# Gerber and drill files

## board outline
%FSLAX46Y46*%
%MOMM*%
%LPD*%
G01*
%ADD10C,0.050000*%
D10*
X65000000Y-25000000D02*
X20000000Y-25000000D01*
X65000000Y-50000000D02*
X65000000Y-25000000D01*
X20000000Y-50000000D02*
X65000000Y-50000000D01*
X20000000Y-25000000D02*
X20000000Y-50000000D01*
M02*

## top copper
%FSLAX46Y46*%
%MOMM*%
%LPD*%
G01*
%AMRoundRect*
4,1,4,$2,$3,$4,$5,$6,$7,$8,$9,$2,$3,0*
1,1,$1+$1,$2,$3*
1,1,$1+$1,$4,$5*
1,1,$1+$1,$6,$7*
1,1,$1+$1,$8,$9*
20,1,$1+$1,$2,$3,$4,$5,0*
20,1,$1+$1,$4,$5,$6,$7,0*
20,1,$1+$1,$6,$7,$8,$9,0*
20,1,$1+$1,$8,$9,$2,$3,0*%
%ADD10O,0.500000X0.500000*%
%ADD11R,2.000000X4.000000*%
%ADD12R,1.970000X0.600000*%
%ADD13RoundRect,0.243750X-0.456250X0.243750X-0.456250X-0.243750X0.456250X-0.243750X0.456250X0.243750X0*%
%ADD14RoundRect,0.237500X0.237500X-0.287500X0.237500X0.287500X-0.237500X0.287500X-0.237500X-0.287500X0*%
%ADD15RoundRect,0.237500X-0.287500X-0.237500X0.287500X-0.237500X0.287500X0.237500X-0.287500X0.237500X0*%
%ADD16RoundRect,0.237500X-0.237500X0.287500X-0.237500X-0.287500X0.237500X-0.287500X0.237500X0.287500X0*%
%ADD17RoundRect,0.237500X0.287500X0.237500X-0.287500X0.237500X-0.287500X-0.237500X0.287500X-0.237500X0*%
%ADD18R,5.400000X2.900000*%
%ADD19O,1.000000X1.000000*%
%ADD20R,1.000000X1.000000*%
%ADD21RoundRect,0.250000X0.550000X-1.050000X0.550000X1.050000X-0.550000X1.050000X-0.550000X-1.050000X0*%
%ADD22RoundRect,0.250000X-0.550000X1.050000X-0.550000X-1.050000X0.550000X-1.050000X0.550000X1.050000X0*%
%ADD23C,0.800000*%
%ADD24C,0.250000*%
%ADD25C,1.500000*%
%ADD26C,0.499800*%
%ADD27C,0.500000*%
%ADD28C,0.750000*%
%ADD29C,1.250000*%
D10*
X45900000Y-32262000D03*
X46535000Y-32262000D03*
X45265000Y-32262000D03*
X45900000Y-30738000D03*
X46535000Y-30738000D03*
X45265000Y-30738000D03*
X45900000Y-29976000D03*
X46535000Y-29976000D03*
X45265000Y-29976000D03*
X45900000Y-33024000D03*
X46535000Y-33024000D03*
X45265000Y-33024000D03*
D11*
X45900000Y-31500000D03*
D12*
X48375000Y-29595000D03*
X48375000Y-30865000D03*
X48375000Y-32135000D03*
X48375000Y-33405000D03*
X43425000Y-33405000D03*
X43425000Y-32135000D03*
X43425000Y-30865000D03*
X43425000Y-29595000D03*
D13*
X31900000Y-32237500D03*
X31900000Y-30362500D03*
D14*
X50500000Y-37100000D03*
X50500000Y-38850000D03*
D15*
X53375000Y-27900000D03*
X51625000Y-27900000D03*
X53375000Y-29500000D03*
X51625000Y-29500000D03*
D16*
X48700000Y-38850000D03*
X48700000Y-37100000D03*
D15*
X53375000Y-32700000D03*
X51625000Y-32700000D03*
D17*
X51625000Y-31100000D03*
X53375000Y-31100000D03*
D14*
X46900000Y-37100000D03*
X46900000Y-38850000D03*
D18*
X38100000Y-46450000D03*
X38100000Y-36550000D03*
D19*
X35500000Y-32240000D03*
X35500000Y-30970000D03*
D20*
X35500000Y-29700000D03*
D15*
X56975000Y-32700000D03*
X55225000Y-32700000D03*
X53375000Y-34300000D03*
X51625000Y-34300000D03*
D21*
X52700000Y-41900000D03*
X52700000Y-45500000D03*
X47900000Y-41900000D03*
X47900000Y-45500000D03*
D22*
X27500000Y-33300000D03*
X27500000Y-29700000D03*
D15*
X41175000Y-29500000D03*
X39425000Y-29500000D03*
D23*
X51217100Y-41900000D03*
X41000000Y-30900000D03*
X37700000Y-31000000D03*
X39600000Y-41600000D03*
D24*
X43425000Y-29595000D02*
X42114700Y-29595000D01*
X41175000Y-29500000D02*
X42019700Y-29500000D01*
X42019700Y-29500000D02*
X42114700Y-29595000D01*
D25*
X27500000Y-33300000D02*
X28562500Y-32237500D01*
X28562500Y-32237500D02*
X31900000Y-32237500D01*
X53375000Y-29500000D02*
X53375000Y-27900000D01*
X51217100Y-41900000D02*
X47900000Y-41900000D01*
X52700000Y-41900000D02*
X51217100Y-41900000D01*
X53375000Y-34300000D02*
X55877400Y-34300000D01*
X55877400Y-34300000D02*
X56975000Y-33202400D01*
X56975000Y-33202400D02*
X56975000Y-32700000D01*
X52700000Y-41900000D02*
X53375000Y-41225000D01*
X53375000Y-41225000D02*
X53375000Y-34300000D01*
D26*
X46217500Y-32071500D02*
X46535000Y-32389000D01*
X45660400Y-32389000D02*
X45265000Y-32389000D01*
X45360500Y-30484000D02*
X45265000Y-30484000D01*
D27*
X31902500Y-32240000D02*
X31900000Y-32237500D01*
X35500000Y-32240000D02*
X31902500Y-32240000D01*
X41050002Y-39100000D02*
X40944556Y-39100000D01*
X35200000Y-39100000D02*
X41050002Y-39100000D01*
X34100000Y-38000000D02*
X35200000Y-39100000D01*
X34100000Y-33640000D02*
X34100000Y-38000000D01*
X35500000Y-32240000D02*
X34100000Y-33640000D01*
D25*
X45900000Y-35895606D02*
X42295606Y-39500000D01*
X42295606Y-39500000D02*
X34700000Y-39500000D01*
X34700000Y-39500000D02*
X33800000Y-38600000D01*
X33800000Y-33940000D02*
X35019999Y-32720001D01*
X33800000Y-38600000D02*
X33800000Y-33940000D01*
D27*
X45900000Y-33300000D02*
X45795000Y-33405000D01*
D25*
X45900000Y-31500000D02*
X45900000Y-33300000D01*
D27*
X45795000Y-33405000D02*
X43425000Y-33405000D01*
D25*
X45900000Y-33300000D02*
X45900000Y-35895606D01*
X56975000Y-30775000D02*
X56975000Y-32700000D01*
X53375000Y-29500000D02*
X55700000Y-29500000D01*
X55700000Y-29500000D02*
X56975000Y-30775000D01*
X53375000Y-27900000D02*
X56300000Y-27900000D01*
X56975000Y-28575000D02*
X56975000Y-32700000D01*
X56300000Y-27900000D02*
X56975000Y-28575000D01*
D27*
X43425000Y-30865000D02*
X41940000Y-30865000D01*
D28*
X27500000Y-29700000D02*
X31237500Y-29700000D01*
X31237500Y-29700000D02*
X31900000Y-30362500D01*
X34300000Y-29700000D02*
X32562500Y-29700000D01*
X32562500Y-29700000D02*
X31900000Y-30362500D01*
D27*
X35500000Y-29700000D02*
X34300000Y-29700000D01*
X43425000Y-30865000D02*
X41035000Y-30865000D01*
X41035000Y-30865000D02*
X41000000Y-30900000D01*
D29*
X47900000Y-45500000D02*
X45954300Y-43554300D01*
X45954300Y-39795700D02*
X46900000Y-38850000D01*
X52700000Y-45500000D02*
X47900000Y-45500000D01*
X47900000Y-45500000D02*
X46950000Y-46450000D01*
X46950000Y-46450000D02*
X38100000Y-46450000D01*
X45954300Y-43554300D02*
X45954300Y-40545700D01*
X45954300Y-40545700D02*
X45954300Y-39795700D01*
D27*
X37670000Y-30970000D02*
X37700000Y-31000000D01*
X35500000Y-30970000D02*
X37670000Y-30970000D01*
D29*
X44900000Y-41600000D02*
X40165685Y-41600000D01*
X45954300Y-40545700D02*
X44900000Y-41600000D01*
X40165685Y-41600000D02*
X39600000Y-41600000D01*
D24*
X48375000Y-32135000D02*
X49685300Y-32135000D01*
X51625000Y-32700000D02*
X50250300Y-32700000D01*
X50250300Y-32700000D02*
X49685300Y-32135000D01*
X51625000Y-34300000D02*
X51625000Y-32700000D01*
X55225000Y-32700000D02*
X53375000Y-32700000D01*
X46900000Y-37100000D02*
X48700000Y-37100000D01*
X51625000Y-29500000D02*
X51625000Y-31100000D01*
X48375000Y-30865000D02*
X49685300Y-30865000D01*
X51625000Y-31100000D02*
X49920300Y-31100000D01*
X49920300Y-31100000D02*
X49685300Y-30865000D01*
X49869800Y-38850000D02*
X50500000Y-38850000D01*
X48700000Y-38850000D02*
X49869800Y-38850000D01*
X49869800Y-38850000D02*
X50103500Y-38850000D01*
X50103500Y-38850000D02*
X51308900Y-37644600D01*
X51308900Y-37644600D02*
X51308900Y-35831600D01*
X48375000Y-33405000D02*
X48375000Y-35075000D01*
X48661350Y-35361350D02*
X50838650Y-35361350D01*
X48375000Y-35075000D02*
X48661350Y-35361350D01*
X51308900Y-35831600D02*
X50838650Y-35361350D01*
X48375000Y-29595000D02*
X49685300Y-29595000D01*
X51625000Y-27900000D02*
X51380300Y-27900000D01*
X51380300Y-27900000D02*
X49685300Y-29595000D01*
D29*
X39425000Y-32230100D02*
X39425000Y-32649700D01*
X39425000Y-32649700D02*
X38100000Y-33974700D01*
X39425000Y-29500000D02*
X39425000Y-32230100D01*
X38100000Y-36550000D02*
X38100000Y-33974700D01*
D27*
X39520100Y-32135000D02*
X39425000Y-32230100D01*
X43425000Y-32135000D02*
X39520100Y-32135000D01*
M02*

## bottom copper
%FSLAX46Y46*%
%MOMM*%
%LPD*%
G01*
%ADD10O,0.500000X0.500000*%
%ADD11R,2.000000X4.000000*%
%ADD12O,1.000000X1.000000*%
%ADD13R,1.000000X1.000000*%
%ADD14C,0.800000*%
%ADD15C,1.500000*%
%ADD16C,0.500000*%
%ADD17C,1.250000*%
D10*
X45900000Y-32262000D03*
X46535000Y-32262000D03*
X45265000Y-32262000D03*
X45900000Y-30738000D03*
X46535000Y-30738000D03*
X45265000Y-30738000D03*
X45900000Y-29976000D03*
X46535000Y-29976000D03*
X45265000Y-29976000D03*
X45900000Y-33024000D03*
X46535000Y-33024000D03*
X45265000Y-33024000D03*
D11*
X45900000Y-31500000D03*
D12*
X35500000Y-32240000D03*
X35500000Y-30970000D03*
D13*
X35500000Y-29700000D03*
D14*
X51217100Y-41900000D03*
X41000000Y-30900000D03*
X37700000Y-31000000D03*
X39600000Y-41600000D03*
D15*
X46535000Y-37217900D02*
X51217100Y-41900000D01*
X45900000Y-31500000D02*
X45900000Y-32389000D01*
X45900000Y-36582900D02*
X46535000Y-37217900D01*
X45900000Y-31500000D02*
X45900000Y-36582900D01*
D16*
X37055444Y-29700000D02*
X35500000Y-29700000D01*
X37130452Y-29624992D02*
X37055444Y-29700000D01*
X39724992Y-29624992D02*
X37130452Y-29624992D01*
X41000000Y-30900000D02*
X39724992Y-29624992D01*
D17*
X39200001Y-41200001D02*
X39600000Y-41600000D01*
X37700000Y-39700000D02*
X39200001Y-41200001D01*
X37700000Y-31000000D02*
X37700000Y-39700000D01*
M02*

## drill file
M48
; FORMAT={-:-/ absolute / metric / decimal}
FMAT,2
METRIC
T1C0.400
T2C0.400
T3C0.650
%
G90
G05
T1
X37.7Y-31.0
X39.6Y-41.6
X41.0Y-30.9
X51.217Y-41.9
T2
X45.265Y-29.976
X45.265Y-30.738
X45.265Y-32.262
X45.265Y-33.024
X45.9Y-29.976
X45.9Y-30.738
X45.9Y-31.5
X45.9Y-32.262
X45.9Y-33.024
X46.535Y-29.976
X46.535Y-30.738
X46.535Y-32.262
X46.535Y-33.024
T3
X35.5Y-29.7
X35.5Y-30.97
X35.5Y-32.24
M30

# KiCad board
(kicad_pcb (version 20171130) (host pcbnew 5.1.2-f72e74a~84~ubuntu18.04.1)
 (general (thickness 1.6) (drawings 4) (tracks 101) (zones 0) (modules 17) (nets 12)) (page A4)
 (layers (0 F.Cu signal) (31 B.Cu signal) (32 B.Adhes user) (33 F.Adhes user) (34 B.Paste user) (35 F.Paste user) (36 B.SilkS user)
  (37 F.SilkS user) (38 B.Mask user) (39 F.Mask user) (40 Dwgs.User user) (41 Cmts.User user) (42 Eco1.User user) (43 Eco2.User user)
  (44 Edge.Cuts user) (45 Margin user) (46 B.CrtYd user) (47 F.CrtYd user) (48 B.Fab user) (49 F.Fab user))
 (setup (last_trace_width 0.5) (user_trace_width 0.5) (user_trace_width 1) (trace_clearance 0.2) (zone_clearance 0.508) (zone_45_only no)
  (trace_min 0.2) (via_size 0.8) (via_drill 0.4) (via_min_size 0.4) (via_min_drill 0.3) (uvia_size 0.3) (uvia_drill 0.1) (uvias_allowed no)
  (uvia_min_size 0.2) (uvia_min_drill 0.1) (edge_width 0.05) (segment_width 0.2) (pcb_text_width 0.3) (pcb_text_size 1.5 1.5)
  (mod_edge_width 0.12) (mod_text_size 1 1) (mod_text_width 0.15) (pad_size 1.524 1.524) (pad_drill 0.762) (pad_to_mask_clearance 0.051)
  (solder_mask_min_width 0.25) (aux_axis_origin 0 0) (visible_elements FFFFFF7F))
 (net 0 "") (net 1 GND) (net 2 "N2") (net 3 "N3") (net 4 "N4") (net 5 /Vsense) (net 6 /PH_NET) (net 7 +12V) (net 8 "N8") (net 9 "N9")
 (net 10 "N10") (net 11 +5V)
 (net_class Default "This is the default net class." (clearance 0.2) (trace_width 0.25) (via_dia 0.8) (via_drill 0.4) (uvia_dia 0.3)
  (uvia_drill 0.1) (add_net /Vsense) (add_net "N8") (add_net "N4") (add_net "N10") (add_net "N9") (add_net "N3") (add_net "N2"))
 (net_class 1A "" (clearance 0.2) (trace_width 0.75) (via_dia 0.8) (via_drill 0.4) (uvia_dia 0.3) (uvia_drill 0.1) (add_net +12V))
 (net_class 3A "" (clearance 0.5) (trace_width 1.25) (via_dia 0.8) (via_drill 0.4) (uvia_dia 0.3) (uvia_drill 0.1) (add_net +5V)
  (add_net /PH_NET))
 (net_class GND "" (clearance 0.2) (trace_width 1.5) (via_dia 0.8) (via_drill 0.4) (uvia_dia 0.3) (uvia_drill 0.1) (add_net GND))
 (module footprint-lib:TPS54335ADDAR (layer F.Cu) (at 45.9 31.5)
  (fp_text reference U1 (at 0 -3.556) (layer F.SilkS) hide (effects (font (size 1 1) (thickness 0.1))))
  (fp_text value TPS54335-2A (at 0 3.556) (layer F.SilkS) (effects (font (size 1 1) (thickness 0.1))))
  (pad PAD thru_hole oval (at 0 0.762) (size 0.5 0.5) (drill 0.4) (layers *.Cu F.Mask) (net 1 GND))
  (pad PAD thru_hole oval (at 0.635 0.762) (size 0.5 0.5) (drill 0.4) (layers *.Cu F.Mask) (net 1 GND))
  (pad PAD thru_hole oval (at -0.635 0.762) (size 0.5 0.5) (drill 0.4) (layers *.Cu F.Mask) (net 1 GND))
  (pad PAD thru_hole oval (at 0 -0.762) (size 0.5 0.5) (drill 0.4) (layers *.Cu F.Mask) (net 1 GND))
  (pad PAD thru_hole oval (at 0.635 -0.762) (size 0.5 0.5) (drill 0.4) (layers *.Cu F.Mask) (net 1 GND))
  (pad PAD thru_hole oval (at -0.635 -0.762) (size 0.5 0.5) (drill 0.4) (layers *.Cu F.Mask) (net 1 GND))
  (pad PAD thru_hole oval (at 0 -1.524) (size 0.5 0.5) (drill 0.4) (layers *.Cu F.Mask) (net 1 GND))
  (pad PAD thru_hole oval (at 0.635 -1.524) (size 0.5 0.5) (drill 0.4) (layers *.Cu F.Mask) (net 1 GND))
  (pad PAD thru_hole oval (at -0.635 -1.524) (size 0.5 0.5) (drill 0.4) (layers *.Cu F.Mask) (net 1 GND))
  (pad PAD thru_hole oval (at 0 1.524) (size 0.5 0.5) (drill 0.4) (layers *.Cu F.Mask) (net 1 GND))
  (pad PAD thru_hole oval (at 0.635 1.524) (size 0.5 0.5) (drill 0.4) (layers *.Cu F.Mask) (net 1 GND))
  (pad PAD thru_hole oval (at -0.635 1.524) (size 0.5 0.5) (drill 0.4) (layers *.Cu F.Mask) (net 1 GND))
  (pad PAD thru_hole rect (at 0 0) (size 2 4) (drill 0.4) (layers *.Cu F.Paste F.Mask) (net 1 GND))
  (pad 8 smd rect (at 2.475 -1.905) (size 1.97 0.6) (layers F.Cu F.Paste F.Mask) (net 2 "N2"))
  (pad 7 smd rect (at 2.475 -0.635) (size 1.97 0.6) (layers F.Cu F.Paste F.Mask) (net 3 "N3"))
  (pad 6 smd rect (at 2.475 0.635) (size 1.97 0.6) (layers F.Cu F.Paste F.Mask) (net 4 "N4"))
  (pad 5 smd rect (at 2.475 1.905) (size 1.97 0.6) (layers F.Cu F.Paste F.Mask) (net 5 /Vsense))
  (pad 4 smd rect (at -2.475 1.905) (size 1.97 0.6) (layers F.Cu F.Paste F.Mask) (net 1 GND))
  (pad 3 smd rect (at -2.475 0.635) (size 1.97 0.6) (layers F.Cu F.Paste F.Mask) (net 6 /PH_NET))
  (pad 2 smd rect (at -2.475 -0.635) (size 1.97 0.6) (layers F.Cu F.Paste F.Mask) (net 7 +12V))
  (pad 1 smd rect (at -2.475 -1.905) (size 1.97 0.6) (layers F.Cu F.Paste F.Mask) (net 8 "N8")))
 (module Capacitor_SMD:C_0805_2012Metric (layer F.Cu) (at 31.9 31.3 270)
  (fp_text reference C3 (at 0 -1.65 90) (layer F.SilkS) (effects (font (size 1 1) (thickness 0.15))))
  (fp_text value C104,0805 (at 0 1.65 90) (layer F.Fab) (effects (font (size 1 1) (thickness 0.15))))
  (pad 2 smd roundrect (at 0.9375 0 270) (size 0.975 1.4) (layers F.Cu F.Paste F.Mask) (roundrect_rratio 0.25) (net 1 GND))
  (pad 1 smd roundrect (at -0.9375 0 270) (size 0.975 1.4) (layers F.Cu F.Paste F.Mask) (roundrect_rratio 0.25) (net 7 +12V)))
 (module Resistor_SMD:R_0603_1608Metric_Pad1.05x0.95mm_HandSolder (layer F.Cu) (at 50.5 37.975 90)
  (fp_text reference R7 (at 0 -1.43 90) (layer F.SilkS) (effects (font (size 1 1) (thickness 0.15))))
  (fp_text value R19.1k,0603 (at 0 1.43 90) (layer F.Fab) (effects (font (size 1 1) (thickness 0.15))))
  (pad 2 smd roundrect (at 0.875 0 90) (size 1.05 0.95) (layers F.Cu F.Paste F.Mask) (roundrect_rratio 0.25) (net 1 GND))
  (pad 1 smd roundrect (at -0.875 0 90) (size 1.05 0.95) (layers F.Cu F.Paste F.Mask) (roundrect_rratio 0.25) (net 5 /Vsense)))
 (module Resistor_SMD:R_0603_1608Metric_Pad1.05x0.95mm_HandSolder (layer F.Cu) (at 52.5 27.9)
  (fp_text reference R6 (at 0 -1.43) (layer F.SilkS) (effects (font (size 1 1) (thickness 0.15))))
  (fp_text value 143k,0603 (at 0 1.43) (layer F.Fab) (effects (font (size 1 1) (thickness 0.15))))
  (pad 2 smd roundrect (at 0.875 0) (size 1.05 0.95) (layers F.Cu F.Paste F.Mask) (roundrect_rratio 0.25) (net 1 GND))
  (pad 1 smd roundrect (at -0.875 0) (size 1.05 0.95) (layers F.Cu F.Paste F.Mask) (roundrect_rratio 0.25) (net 2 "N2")))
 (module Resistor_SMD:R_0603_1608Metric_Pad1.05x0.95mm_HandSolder (layer F.Cu) (at 52.5 29.5)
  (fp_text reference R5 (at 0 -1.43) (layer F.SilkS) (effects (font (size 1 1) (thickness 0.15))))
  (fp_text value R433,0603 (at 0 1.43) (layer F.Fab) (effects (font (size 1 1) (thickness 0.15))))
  (pad 2 smd roundrect (at 0.875 0) (size 1.05 0.95) (layers F.Cu F.Paste F.Mask) (roundrect_rratio 0.25) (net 1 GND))
  (pad 1 smd roundrect (at -0.875 0) (size 1.05 0.95) (layers F.Cu F.Paste F.Mask) (roundrect_rratio 0.25) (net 3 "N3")))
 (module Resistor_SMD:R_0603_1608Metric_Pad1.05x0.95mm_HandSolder (layer F.Cu) (at 48.7 37.975 270)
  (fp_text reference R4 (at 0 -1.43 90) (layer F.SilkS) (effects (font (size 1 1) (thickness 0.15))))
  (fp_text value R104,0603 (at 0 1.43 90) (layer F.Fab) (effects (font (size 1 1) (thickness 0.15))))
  (pad 2 smd roundrect (at 0.875 0 270) (size 1.05 0.95) (layers F.Cu F.Paste F.Mask) (roundrect_rratio 0.25) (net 5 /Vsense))
  (pad 1 smd roundrect (at -0.875 0 270) (size 1.05 0.95) (layers F.Cu F.Paste F.Mask) (roundrect_rratio 0.25) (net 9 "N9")))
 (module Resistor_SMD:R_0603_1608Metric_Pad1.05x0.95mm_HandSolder (layer F.Cu) (at 52.5 32.7)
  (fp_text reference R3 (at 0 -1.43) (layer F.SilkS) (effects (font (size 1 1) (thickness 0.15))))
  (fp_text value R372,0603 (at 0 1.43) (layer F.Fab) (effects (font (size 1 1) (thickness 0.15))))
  (pad 2 smd roundrect (at 0.875 0) (size 1.05 0.95) (layers F.Cu F.Paste F.Mask) (roundrect_rratio 0.25) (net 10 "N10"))
  (pad 1 smd roundrect (at -0.875 0) (size 1.05 0.95) (layers F.Cu F.Paste F.Mask) (roundrect_rratio 0.25) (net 4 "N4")))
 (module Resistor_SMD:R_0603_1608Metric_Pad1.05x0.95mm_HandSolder (layer F.Cu) (at 52.5 31.1 180)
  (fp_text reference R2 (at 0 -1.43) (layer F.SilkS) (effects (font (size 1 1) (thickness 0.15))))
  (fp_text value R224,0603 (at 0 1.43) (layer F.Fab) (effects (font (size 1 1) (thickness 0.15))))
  (pad 2 smd roundrect (at 0.875 0 180) (size 1.05 0.95) (layers F.Cu F.Paste F.Mask) (roundrect_rratio 0.25) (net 3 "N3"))
  (pad 1 smd roundrect (at -0.875 0 180) (size 1.05 0.95) (layers F.Cu F.Paste F.Mask) (roundrect_rratio 0.25) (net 7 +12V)))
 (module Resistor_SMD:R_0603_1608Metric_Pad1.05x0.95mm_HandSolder (layer F.Cu) (at 46.9 37.975 90)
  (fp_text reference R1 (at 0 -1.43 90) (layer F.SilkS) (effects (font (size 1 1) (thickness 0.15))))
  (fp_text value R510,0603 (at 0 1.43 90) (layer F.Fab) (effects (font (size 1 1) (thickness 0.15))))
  (pad 2 smd roundrect (at 0.875 0 90) (size 1.05 0.95) (layers F.Cu F.Paste F.Mask) (roundrect_rratio 0.25) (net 9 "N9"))
  (pad 1 smd roundrect (at -0.875 0 90) (size 1.05 0.95) (layers F.Cu F.Paste F.Mask) (roundrect_rratio 0.25) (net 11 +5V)))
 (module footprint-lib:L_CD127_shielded (layer F.Cu) (at 38.1 41.5 270)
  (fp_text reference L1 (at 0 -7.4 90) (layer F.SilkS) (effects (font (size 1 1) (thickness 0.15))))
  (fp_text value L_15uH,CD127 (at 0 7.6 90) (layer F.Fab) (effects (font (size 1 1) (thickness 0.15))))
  (pad 2 smd rect (at 4.95 0 270) (size 2.9 5.4) (layers F.Cu F.Paste F.Mask) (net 11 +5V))
  (pad 1 smd rect (at -4.95 0 270) (size 2.9 5.4) (layers F.Cu F.Paste F.Mask) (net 6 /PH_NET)))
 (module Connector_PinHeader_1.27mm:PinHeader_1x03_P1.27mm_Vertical (layer F.Cu) (at 35.5 29.7)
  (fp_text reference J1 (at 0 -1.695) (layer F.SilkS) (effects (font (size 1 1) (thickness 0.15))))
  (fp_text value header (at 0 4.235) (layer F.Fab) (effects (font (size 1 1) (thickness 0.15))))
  (pad 3 thru_hole oval (at 0 2.54) (size 1 1) (drill 0.65) (layers *.Cu *.Mask) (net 1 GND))
  (pad 2 thru_hole oval (at 0 1.27) (size 1 1) (drill 0.65) (layers *.Cu *.Mask) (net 11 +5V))
  (pad 1 thru_hole rect (at 0 0) (size 1 1) (drill 0.65) (layers *.Cu *.Mask) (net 7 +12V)))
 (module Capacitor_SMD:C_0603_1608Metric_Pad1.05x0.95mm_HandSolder (layer F.Cu) (at 56.1 32.7)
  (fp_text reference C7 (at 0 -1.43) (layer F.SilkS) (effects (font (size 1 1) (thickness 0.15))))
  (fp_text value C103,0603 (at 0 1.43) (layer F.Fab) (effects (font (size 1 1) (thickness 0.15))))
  (pad 2 smd roundrect (at 0.875 0) (size 1.05 0.95) (layers F.Cu F.Paste F.Mask) (roundrect_rratio 0.25) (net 1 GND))
  (pad 1 smd roundrect (at -0.875 0) (size 1.05 0.95) (layers F.Cu F.Paste F.Mask) (roundrect_rratio 0.25) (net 10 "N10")))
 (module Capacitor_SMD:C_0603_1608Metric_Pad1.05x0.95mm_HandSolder (layer F.Cu) (at 52.5 34.3)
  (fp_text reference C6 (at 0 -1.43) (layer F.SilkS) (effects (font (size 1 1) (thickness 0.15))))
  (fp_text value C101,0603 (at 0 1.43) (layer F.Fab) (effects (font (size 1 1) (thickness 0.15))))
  (pad 2 smd roundrect (at 0.875 0) (size 1.05 0.95) (layers F.Cu F.Paste F.Mask) (roundrect_rratio 0.25) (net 1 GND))
  (pad 1 smd roundrect (at -0.875 0) (size 1.05 0.95) (layers F.Cu F.Paste F.Mask) (roundrect_rratio 0.25) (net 4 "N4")))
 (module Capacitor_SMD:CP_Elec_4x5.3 (layer F.Cu) (at 52.7 43.7 90)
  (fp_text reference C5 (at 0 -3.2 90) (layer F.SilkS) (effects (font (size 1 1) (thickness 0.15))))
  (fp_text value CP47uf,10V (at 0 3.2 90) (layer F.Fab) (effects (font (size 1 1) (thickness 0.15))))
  (pad 2 smd roundrect (at 1.8 0 90) (size 2.6 1.6) (layers F.Cu F.Paste F.Mask) (roundrect_rratio 0.15625) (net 1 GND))
  (pad 1 smd roundrect (at -1.8 0 90) (size 2.6 1.6) (layers F.Cu F.Paste F.Mask) (roundrect_rratio 0.15625) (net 11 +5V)))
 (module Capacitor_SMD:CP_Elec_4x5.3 (layer F.Cu) (at 47.9 43.7 90)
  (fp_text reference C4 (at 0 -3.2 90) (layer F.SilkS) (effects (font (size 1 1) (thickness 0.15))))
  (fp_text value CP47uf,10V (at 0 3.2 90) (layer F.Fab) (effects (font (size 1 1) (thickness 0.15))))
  (pad 2 smd roundrect (at 1.8 0 90) (size 2.6 1.6) (layers F.Cu F.Paste F.Mask) (roundrect_rratio 0.15625) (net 1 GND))
  (pad 1 smd roundrect (at -1.8 0 90) (size 2.6 1.6) (layers F.Cu F.Paste F.Mask) (roundrect_rratio 0.15625) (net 11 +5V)))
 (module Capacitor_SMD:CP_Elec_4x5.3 (layer F.Cu) (at 27.5 31.5 270)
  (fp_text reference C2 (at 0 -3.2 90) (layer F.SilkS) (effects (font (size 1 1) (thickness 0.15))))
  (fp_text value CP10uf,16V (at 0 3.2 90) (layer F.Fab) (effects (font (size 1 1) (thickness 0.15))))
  (pad 2 smd roundrect (at 1.8 0 270) (size 2.6 1.6) (layers F.Cu F.Paste F.Mask) (roundrect_rratio 0.15625) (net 1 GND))
  (pad 1 smd roundrect (at -1.8 0 270) (size 2.6 1.6) (layers F.Cu F.Paste F.Mask) (roundrect_rratio 0.15625) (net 7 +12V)))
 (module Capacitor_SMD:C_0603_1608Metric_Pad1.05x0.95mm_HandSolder (layer F.Cu) (at 40.3 29.5)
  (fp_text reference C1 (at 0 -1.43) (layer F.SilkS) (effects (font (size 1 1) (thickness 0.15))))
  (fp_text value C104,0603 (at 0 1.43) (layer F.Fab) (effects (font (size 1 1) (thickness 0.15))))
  (pad 2 smd roundrect (at 0.875 0) (size 1.05 0.95) (layers F.Cu F.Paste F.Mask) (roundrect_rratio 0.25) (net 8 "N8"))
  (pad 1 smd roundrect (at -0.875 0) (size 1.05 0.95) (layers F.Cu F.Paste F.Mask) (roundrect_rratio 0.25) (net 6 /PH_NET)))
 (gr_line (start 65 25) (end 20 25) (layer Edge.Cuts) (width 0.05))
 (gr_line (start 65 50) (end 65 25) (layer Edge.Cuts) (width 0.05))
 (gr_line (start 20 50) (end 65 50) (layer Edge.Cuts) (width 0.05))
 (gr_line (start 20 25) (end 20 50) (layer Edge.Cuts) (width 0.05))
 (segment (start 43.425 29.595) (end 42.1147 29.595) (width 0.25) (layer F.Cu) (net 8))
 (segment (start 41.175 29.5) (end 42.0197 29.5) (width 0.25) (layer F.Cu) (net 8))
 (segment (start 42.0197 29.5) (end 42.1147 29.595) (width 0.25) (layer F.Cu) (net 8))
 (segment (start 27.5 33.3) (end 28.5625 32.2375) (width 1.5) (layer F.Cu) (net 1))
 (segment (start 28.5625 32.2375) (end 31.9 32.2375) (width 1.5) (layer F.Cu) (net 1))
 (segment (start 53.375 29.5) (end 53.375 27.9) (width 1.5) (layer F.Cu) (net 1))
 (segment (start 46.535 37.2179) (end 51.2171 41.9) (width 1.5) (layer B.Cu) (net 1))
 (segment (start 51.2171 41.9) (end 47.9 41.9) (width 1.5) (layer F.Cu) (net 1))
 (segment (start 52.7 41.9) (end 51.2171 41.9) (width 1.5) (layer F.Cu) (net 1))
 (segment (start 53.375 34.3) (end 55.8774 34.3) (width 1.5) (layer F.Cu) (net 1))
 (segment (start 55.8774 34.3) (end 56.975 33.2024) (width 1.5) (layer F.Cu) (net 1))
 (segment (start 56.975 33.2024) (end 56.975 32.7) (width 1.5) (layer F.Cu) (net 1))
 (segment (start 52.7 41.9) (end 53.375 41.225) (width 1.5) (layer F.Cu) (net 1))
 (segment (start 53.375 41.225) (end 53.375 34.3) (width 1.5) (layer F.Cu) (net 1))
 (segment (start 46.2175 32.0715) (end 46.535 32.389) (width 0.4998) (layer F.Cu) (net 1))
 (segment (start 45.6604 32.389) (end 45.265 32.389) (width 0.4998) (layer F.Cu) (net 1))
 (segment (start 45.3605 30.484) (end 45.265 30.484) (width 0.4998) (layer F.Cu) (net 1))
 (segment (start 45.9 31.5) (end 45.9 32.389) (width 1.5) (layer B.Cu) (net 1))
 (via (at 51.2171 41.9) (size 0.8) (layers F.Cu B.Cu) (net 1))
 (segment (start 45.9 36.5829) (end 46.535 37.2179) (width 1.5) (layer B.Cu) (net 1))
 (segment (start 45.9 31.5) (end 45.9 36.5829) (width 1.5) (layer B.Cu) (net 1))
 (segment (start 31.9025 32.24) (end 31.9 32.2375) (width 0.5) (layer F.Cu) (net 1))
 (segment (start 35.5 32.24) (end 31.9025 32.24) (width 0.5) (layer F.Cu) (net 1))
 (segment (start 41.050002 39.1) (end 40.944556 39.1) (width 0.5) (layer F.Cu) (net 1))
 (segment (start 35.2 39.1) (end 41.050002 39.1) (width 0.5) (layer F.Cu) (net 1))
 (segment (start 34.1 38) (end 35.2 39.1) (width 0.5) (layer F.Cu) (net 1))
 (segment (start 34.1 33.64) (end 34.1 38) (width 0.5) (layer F.Cu) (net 1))
 (segment (start 35.5 32.24) (end 34.1 33.64) (width 0.5) (layer F.Cu) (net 1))
 (segment (start 45.9 35.895606) (end 42.295606 39.5) (width 1.5) (layer F.Cu) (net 1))
 (segment (start 42.295606 39.5) (end 34.7 39.5) (width 1.5) (layer F.Cu) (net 1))
 (segment (start 34.7 39.5) (end 33.8 38.6) (width 1.5) (layer F.Cu) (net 1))
 (segment (start 33.8 33.94) (end 35.019999 32.720001) (width 1.5) (layer F.Cu) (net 1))
 (segment (start 33.8 38.6) (end 33.8 33.94) (width 1.5) (layer F.Cu) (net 1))
 (segment (start 45.9 33.3) (end 45.795 33.405) (width 0.5) (layer F.Cu) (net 1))
 (segment (start 45.9 31.5) (end 45.9 33.3) (width 1.5) (layer F.Cu) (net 1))
 (segment (start 45.795 33.405) (end 43.425 33.405) (width 0.5) (layer F.Cu) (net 1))
 (segment (start 45.9 33.3) (end 45.9 35.895606) (width 1.5) (layer F.Cu) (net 1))
 (segment (start 56.975 30.775) (end 56.975 32.7) (width 1.5) (layer F.Cu) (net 1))
 (segment (start 53.375 29.5) (end 55.7 29.5) (width 1.5) (layer F.Cu) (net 1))
 (segment (start 55.7 29.5) (end 56.975 30.775) (width 1.5) (layer F.Cu) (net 1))
 (segment (start 53.375 27.9) (end 56.3 27.9) (width 1.5) (layer F.Cu) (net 1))
 (segment (start 56.975 28.575) (end 56.975 32.7) (width 1.5) (layer F.Cu) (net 1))
 (segment (start 56.3 27.9) (end 56.975 28.575) (width 1.5) (layer F.Cu) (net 1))
 (segment (start 43.425 30.865) (end 41.94 30.865) (width 0.5) (layer F.Cu) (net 7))
 (segment (start 27.5 29.7) (end 31.2375 29.7) (width 0.75) (layer F.Cu) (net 7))
 (segment (start 31.2375 29.7) (end 31.9 30.3625) (width 0.75) (layer F.Cu) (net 7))
 (segment (start 34.3 29.7) (end 32.5625 29.7) (width 0.75) (layer F.Cu) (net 7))
 (segment (start 32.5625 29.7) (end 31.9 30.3625) (width 0.75) (layer F.Cu) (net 7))
 (segment (start 35.5 29.7) (end 34.3 29.7) (width 0.5) (layer F.Cu) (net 7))
 (via (at 41 30.9) (size 0.8) (drill 0.4) (layers F.Cu B.Cu) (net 7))
 (segment (start 43.425 30.865) (end 41.035 30.865) (width 0.5) (layer F.Cu) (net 7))
 (segment (start 41.035 30.865) (end 41 30.9) (width 0.5) (layer F.Cu) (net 7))
 (segment (start 37.055444 29.7) (end 35.5 29.7) (width 0.5) (layer B.Cu) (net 7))
 (segment (start 37.130452 29.624992) (end 37.055444 29.7) (width 0.5) (layer B.Cu) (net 7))
 (segment (start 39.724992 29.624992) (end 37.130452 29.624992) (width 0.5) (layer B.Cu) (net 7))
 (segment (start 41 30.9) (end 39.724992 29.624992) (width 0.5) (layer B.Cu) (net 7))
 (segment (start 47.9 45.5) (end 45.9543 43.5543) (width 1.25) (layer F.Cu) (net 11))
 (segment (start 45.9543 39.7957) (end 46.9 38.85) (width 1.25) (layer F.Cu) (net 11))
 (segment (start 52.7 45.5) (end 47.9 45.5) (width 1.25) (layer F.Cu) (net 11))
 (segment (start 47.9 45.5) (end 46.95 46.45) (width 1.25) (layer F.Cu) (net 11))
 (segment (start 46.95 46.45) (end 38.1 46.45) (width 1.25) (layer F.Cu) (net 11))
 (segment (start 45.9543 43.5543) (end 45.9543 40.5457) (width 1.25) (layer F.Cu) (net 11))
 (segment (start 45.9543 40.5457) (end 45.9543 39.7957) (width 1.25) (layer F.Cu) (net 11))
 (via (at 37.7 31) (size 0.8) (drill 0.4) (layers F.Cu B.Cu) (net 11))
 (segment (start 37.67 30.97) (end 37.7 31) (width 0.5) (layer F.Cu) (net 11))
 (segment (start 35.5 30.97) (end 37.67 30.97) (width 0.5) (layer F.Cu) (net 11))
 (segment (start 39.200001 41.200001) (end 39.6 41.6) (width 1.25) (layer B.Cu) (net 11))
 (segment (start 37.7 39.7) (end 39.200001 41.200001) (width 1.25) (layer B.Cu) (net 11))
 (segment (start 37.7 31) (end 37.7 39.7) (width 1.25) (layer B.Cu) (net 11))
 (segment (start 44.9 41.6) (end 40.165685 41.6) (width 1.25) (layer F.Cu) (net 11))
 (via (at 39.6 41.6) (size 0.8) (drill 0.4) (layers F.Cu B.Cu) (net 11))
 (segment (start 45.9543 40.5457) (end 44.9 41.6) (width 1.25) (layer F.Cu) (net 11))
 (segment (start 40.165685 41.6) (end 39.6 41.6) (width 1.25) (layer F.Cu) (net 11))
 (segment (start 48.375 32.135) (end 49.6853 32.135) (width 0.25) (layer F.Cu) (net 4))
 (segment (start 51.625 32.7) (end 50.2503 32.7) (width 0.25) (layer F.Cu) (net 4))
 (segment (start 50.2503 32.7) (end 49.6853 32.135) (width 0.25) (layer F.Cu) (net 4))
 (segment (start 51.625 34.3) (end 51.625 32.7) (width 0.25) (layer F.Cu) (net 4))
 (segment (start 55.225 32.7) (end 53.375 32.7) (width 0.25) (layer F.Cu) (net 10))
 (segment (start 46.9 37.1) (end 48.7 37.1) (width 0.25) (layer F.Cu) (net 9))
 (segment (start 51.625 29.5) (end 51.625 31.1) (width 0.25) (layer F.Cu) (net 3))
 (segment (start 48.375 30.865) (end 49.6853 30.865) (width 0.25) (layer F.Cu) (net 3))
 (segment (start 51.625 31.1) (end 49.9203 31.1) (width 0.25) (layer F.Cu) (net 3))
 (segment (start 49.9203 31.1) (end 49.6853 30.865) (width 0.25) (layer F.Cu) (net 3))
 (segment (start 49.8698 38.85) (end 50.5 38.85) (width 0.25) (layer F.Cu) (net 5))
 (segment (start 48.7 38.85) (end 49.8698 38.85) (width 0.25) (layer F.Cu) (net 5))
 (segment (start 49.8698 38.85) (end 50.1035 38.85) (width 0.25) (layer F.Cu) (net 5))
 (segment (start 50.1035 38.85) (end 51.3089 37.6446) (width 0.25) (layer F.Cu) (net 5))
 (segment (start 51.3089 37.6446) (end 51.3089 35.8316) (width 0.25) (layer F.Cu) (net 5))
 (segment (start 48.375 33.405) (end 48.375 35.075) (width 0.25) (layer F.Cu) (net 5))
 (segment (start 48.66135 35.36135) (end 50.83865 35.36135) (width 0.25) (layer F.Cu) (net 5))
 (segment (start 48.375 35.075) (end 48.66135 35.36135) (width 0.25) (layer F.Cu) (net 5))
 (segment (start 51.3089 35.8316) (end 50.83865 35.36135) (width 0.25) (layer F.Cu) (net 5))
 (segment (start 48.375 29.595) (end 49.6853 29.595) (width 0.25) (layer F.Cu) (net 2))
 (segment (start 51.625 27.9) (end 51.3803 27.9) (width 0.25) (layer F.Cu) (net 2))
 (segment (start 51.3803 27.9) (end 49.6853 29.595) (width 0.25) (layer F.Cu) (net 2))
 (segment (start 39.425 32.2301) (end 39.425 32.6497) (width 1.25) (layer F.Cu) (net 6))
 (segment (start 39.425 32.6497) (end 38.1 33.9747) (width 1.25) (layer F.Cu) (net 6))
 (segment (start 39.425 29.5) (end 39.425 32.2301) (width 1.25) (layer F.Cu) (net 6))
 (segment (start 38.1 36.55) (end 38.1 33.9747) (width 1.25) (layer F.Cu) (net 6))
 (segment (start 39.5201 32.135) (end 39.425 32.2301) (width 0.5) (layer F.Cu) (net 6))
 (segment (start 43.425 32.135) (end 39.5201 32.135) (width 0.5) (layer F.Cu) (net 6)))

